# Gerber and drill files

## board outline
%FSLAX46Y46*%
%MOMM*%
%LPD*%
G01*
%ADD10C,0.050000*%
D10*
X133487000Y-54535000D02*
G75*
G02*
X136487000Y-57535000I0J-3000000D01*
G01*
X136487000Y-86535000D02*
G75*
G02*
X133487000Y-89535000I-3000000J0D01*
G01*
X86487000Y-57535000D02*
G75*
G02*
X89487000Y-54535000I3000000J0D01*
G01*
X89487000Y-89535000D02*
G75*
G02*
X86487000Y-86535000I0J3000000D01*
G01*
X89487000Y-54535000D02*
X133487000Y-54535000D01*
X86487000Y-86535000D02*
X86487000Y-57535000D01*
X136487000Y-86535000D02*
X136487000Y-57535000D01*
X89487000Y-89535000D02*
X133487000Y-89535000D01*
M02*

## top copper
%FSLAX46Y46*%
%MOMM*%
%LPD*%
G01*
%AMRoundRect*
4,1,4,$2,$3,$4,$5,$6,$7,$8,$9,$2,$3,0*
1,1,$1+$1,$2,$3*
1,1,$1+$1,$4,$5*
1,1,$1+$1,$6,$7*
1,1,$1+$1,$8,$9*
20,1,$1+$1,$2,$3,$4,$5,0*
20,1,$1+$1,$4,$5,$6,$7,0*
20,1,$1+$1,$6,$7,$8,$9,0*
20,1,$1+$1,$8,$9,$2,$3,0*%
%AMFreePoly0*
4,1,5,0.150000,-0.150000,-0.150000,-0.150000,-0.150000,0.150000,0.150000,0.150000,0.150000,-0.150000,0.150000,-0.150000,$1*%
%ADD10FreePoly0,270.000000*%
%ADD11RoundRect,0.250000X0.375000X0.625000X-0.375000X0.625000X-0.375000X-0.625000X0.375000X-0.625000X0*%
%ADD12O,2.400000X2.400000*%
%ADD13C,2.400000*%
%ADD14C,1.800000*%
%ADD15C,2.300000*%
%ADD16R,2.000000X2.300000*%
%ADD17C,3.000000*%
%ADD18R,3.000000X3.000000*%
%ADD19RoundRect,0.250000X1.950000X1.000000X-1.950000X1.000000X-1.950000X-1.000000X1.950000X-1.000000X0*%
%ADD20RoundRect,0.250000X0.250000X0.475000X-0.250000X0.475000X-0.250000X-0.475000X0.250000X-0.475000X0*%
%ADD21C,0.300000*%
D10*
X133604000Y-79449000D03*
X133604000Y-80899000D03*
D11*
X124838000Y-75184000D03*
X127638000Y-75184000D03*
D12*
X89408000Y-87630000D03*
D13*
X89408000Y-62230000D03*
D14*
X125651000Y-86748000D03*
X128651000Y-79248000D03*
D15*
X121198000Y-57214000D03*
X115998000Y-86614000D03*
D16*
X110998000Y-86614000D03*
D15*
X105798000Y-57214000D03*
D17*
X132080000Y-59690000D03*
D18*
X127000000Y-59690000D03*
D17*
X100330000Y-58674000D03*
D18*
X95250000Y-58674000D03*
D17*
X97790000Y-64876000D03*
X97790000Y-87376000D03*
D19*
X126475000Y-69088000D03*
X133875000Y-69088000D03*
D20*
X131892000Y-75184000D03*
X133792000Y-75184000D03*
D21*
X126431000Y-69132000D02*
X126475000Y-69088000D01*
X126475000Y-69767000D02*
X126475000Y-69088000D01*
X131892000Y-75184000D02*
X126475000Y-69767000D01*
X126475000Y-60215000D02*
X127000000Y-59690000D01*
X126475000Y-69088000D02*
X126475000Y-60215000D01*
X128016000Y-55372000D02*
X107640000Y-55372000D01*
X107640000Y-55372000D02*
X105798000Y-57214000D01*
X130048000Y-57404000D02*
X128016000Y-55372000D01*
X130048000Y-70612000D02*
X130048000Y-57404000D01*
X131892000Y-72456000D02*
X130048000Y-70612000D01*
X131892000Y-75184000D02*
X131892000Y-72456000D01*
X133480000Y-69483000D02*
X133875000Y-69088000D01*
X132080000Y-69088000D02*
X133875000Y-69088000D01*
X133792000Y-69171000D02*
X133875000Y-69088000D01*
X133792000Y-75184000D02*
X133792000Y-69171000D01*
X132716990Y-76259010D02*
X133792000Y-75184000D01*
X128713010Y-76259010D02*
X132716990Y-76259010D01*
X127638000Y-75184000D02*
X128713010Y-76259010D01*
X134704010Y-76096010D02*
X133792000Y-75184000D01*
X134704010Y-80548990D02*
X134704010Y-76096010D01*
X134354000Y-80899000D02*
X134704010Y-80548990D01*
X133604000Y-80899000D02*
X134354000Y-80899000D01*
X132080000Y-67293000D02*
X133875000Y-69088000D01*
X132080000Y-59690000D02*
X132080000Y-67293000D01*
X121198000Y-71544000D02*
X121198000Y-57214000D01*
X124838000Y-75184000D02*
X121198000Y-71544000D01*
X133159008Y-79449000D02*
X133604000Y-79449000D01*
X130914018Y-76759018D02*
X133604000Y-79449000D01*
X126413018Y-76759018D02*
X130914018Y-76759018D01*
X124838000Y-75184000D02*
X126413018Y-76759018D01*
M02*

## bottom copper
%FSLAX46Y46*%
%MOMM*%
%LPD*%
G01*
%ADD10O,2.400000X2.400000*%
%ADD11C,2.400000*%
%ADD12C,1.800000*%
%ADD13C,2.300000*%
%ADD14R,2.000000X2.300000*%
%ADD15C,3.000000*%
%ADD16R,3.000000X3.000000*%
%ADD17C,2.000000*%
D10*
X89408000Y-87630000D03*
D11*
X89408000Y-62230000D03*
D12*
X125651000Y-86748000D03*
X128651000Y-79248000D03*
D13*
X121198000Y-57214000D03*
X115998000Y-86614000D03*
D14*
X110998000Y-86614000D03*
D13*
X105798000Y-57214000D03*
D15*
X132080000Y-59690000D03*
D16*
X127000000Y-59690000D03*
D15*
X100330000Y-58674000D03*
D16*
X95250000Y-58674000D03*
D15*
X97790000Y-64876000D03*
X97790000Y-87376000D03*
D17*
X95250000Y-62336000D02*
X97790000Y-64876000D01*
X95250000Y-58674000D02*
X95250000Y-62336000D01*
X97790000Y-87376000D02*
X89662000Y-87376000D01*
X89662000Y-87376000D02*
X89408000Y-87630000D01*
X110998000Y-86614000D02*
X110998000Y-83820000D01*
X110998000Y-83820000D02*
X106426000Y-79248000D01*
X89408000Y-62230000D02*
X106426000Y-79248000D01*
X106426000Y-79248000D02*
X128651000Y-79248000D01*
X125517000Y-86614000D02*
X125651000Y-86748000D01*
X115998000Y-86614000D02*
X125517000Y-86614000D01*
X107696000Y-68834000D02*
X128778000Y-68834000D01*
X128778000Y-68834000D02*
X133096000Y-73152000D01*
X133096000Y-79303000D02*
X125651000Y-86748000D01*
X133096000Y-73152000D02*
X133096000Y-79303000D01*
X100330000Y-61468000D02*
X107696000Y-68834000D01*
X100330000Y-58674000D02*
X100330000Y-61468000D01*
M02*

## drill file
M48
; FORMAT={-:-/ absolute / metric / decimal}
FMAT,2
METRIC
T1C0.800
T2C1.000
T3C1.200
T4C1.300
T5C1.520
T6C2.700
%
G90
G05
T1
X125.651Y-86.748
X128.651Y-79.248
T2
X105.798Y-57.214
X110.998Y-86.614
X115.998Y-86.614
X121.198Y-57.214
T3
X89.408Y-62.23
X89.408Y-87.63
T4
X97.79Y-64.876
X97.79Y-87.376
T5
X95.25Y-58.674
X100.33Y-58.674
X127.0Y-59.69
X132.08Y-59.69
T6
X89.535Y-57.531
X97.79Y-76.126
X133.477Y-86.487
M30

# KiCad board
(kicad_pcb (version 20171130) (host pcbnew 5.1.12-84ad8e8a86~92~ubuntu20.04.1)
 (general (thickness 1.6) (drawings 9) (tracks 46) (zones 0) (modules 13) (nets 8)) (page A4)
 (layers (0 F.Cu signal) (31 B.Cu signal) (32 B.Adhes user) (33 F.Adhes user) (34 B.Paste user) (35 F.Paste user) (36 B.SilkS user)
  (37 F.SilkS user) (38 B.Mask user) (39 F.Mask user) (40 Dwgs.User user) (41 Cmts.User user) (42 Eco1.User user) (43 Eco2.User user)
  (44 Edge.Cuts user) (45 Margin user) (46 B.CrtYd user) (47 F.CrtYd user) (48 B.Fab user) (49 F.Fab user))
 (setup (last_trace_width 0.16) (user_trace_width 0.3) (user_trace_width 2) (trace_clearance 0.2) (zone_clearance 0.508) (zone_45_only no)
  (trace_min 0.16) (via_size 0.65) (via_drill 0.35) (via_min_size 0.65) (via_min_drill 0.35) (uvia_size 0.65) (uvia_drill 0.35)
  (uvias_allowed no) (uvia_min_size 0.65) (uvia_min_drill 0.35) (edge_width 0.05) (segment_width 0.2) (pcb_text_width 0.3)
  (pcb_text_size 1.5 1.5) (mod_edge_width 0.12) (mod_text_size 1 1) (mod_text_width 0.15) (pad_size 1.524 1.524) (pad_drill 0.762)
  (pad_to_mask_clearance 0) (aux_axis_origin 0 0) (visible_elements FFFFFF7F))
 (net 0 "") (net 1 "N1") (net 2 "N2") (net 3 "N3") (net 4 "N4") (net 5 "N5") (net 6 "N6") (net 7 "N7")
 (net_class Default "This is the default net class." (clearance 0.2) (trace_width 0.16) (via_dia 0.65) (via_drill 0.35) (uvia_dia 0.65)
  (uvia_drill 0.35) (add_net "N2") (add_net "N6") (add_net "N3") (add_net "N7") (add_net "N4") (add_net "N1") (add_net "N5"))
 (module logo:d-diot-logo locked (layer B.Cu) (at 112.522 69.596 180)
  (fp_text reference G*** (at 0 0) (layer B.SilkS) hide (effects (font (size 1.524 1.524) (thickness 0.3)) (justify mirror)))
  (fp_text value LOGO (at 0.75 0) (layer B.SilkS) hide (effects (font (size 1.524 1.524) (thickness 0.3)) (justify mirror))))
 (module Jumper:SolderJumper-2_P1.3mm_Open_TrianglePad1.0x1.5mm (layer F.Cu) (at 133.604 80.174 270)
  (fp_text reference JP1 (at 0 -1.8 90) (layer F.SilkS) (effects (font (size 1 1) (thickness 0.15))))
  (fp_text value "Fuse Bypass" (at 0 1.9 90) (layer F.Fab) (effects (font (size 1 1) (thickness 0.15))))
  (pad 1 smd custom (at -0.725 0 270) (size 0.3 0.3) (layers F.Cu F.Mask) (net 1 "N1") (zone_connect 2)
   (options (clearance outline) (anchor rect)) (primitives))
  (pad 2 smd custom (at 0.725 0 270) (size 0.3 0.3) (layers F.Cu F.Mask) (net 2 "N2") (zone_connect 2)
   (options (clearance outline) (anchor rect)) (primitives)))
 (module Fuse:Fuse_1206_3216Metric (layer F.Cu) (at 126.238 75.184 180)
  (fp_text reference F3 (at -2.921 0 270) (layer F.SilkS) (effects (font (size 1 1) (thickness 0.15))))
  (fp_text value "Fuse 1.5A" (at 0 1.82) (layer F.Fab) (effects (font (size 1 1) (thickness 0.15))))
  (pad 2 smd roundrect (at 1.4 0 180) (size 1.25 1.75) (layers F.Cu F.Paste F.Mask) (roundrect_rratio 0.2) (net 1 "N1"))
  (pad 1 smd roundrect (at -1.4 0 180) (size 1.25 1.75) (layers F.Cu F.Paste F.Mask) (roundrect_rratio 0.2) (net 2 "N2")))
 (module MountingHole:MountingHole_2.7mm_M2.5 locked (layer F.Cu) (at 133.477 86.487 90)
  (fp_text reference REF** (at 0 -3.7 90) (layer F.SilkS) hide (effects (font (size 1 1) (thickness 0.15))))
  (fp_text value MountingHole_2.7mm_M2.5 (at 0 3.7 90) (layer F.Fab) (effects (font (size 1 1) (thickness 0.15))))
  (pad 1 np_thru_hole circle (at 0 0 90) (size 2.7 2.7) (drill 2.7) (layers *.Cu *.Mask)))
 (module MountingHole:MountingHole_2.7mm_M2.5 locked (layer F.Cu) (at 89.535 57.531 90)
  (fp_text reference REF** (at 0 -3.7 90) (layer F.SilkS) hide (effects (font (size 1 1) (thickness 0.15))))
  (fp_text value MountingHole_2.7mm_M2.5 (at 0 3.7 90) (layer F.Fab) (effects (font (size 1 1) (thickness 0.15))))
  (pad 1 np_thru_hole circle (at 0 0 90) (size 2.7 2.7) (drill 2.7) (layers *.Cu *.Mask)))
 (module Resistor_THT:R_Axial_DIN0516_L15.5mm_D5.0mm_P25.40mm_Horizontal (layer F.Cu) (at 89.408 62.23 270)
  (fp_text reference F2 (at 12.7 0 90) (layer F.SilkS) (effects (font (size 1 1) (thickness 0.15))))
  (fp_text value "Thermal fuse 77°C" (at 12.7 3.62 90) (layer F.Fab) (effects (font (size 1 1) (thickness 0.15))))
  (pad 2 thru_hole oval (at 25.4 0 270) (size 2.4 2.4) (drill 1.2) (layers *.Cu *.Mask) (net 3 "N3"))
  (pad 1 thru_hole circle (at 0 0 270) (size 2.4 2.4) (drill 1.2) (layers *.Cu *.Mask) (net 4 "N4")))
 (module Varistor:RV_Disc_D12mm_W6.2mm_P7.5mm (layer F.Cu) (at 128.651 79.248 270)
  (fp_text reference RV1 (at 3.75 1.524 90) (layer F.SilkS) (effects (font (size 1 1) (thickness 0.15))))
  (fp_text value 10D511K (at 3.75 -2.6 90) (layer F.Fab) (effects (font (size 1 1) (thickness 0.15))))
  (pad 2 thru_hole circle (at 7.5 3 270) (size 1.8 1.8) (drill 0.8) (layers *.Cu *.Mask) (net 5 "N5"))
  (pad 1 thru_hole circle (at 0 0 270) (size 1.8 1.8) (drill 0.8) (layers *.Cu *.Mask) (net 4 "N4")))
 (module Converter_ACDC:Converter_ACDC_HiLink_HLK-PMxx (layer F.Cu) (at 110.998 86.614 90)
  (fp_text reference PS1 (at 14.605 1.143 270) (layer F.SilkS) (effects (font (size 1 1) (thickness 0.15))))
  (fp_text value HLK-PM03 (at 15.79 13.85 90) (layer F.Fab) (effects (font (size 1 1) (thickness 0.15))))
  (pad 4 thru_hole circle (at 29.4 10.2 90) (size 2.3 2.3) (drill 1) (layers *.Cu *.Mask) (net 1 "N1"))
  (pad 2 thru_hole circle (at 0 5 90) (size 2.3 2.3) (drill 1) (layers *.Cu *.Mask) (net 5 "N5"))
  (pad 1 thru_hole rect (at 0 0 90) (size 2.3 2) (drill 1) (layers *.Cu *.Mask) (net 4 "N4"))
  (pad 3 thru_hole circle (at 29.4 -5.2 90) (size 2.3 2.3) (drill 1) (layers *.Cu *.Mask) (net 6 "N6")))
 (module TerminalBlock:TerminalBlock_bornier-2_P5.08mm (layer F.Cu) (at 127 59.69)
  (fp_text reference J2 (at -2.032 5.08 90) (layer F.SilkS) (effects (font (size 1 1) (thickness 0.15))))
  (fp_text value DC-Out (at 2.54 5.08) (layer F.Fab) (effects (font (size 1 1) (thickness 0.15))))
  (pad 2 thru_hole circle (at 5.08 0) (size 3 3) (drill 1.52) (layers *.Cu *.Mask) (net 2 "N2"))
  (pad 1 thru_hole rect (at 0 0) (size 3 3) (drill 1.52) (layers *.Cu *.Mask) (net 6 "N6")))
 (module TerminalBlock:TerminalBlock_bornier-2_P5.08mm (layer F.Cu) (at 95.25 58.674)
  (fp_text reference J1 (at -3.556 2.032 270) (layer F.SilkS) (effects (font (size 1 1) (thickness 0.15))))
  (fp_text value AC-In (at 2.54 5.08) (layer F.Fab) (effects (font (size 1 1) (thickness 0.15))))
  (pad 2 thru_hole circle (at 5.08 0) (size 3 3) (drill 1.52) (layers *.Cu *.Mask) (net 5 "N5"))
  (pad 1 thru_hole rect (at 0 0) (size 3 3) (drill 1.52) (layers *.Cu *.Mask) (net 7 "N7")))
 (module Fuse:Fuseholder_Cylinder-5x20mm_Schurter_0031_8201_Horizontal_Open (layer F.Cu) (at 97.79 87.376 90)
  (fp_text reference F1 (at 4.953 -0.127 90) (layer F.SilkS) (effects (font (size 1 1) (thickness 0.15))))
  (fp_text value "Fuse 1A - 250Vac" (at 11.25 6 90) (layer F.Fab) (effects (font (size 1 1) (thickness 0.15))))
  (pad "" np_thru_hole circle (at 11.25 0 90) (size 2.7 2.7) (drill 2.7) (layers *.Cu *.Mask))
  (pad 2 thru_hole circle (at 22.5 0 90) (size 3 3) (drill 1.3) (layers *.Cu *.Mask) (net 7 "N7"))
  (pad 1 thru_hole circle (at 0 0 90) (size 3 3) (drill 1.3) (layers *.Cu *.Mask) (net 3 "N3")))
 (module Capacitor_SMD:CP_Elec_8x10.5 (layer F.Cu) (at 130.175 69.088 180)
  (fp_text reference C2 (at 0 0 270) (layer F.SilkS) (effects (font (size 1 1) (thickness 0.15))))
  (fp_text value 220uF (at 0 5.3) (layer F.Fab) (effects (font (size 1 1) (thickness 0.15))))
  (pad 2 smd roundrect (at 3.7 0 180) (size 4.4 2.5) (layers F.Cu F.Paste F.Mask) (roundrect_rratio 0.1) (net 6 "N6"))
  (pad 1 smd roundrect (at -3.7 0 180) (size 4.4 2.5) (layers F.Cu F.Paste F.Mask) (roundrect_rratio 0.1) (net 2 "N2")))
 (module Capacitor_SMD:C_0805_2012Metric (layer F.Cu) (at 132.842 75.184 180)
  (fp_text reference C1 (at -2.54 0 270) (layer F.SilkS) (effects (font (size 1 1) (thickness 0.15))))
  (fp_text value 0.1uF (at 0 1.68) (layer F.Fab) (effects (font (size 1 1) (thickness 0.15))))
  (pad 2 smd roundrect (at 0.95 0 180) (size 1 1.45) (layers F.Cu F.Paste F.Mask) (roundrect_rratio 0.25) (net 6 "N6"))
  (pad 1 smd roundrect (at -0.95 0 180) (size 1 1.45) (layers F.Cu F.Paste F.Mask) (roundrect_rratio 0.25) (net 2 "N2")))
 (gr_arc (start 133.487 57.535) (end 136.487 57.535) (angle -90) (layer Edge.Cuts) (width 0.05))
 (gr_arc (start 133.487 86.535) (end 133.487 89.535) (angle -90) (layer Edge.Cuts) (width 0.05))
 (gr_arc (start 89.487 57.535) (end 89.487 54.535) (angle -90) (layer Edge.Cuts) (width 0.05))
 (gr_arc (start 89.487 86.535) (end 86.487 86.535) (angle -90) (layer Edge.Cuts) (width 0.05))
 (gr_line (start 89.487 54.535) (end 133.487 54.535) (layer Edge.Cuts) (width 0.05))
 (gr_line (start 86.487 86.535) (end 86.487 57.535) (layer Edge.Cuts) (width 0.05))
 (gr_line (start 136.487 86.535) (end 136.487 57.535) (layer Edge.Cuts) (width 0.05))
 (gr_line (start 89.487 89.535) (end 133.487 89.535) (layer Edge.Cuts) (width 0.05))
 (segment (start 126.431 69.132) (end 126.475 69.088) (width 0.3) (layer F.Cu) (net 6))
 (segment (start 126.475 69.767) (end 126.475 69.088) (width 0.3) (layer F.Cu) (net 6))
 (segment (start 131.892 75.184) (end 126.475 69.767) (width 0.3) (layer F.Cu) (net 6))
 (segment (start 126.475 60.215) (end 127 59.69) (width 0.3) (layer F.Cu) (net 6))
 (segment (start 126.475 69.088) (end 126.475 60.215) (width 0.3) (layer F.Cu) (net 6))
 (segment (start 128.016 55.372) (end 107.64 55.372) (width 0.3) (layer F.Cu) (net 6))
 (segment (start 107.64 55.372) (end 105.798 57.214) (width 0.3) (layer F.Cu) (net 6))
 (segment (start 130.048 57.404) (end 128.016 55.372) (width 0.3) (layer F.Cu) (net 6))
 (segment (start 130.048 70.612) (end 130.048 57.404) (width 0.3) (layer F.Cu) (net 6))
 (segment (start 131.892 72.456) (end 130.048 70.612) (width 0.3) (layer F.Cu) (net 6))
 (segment (start 131.892 75.184) (end 131.892 72.456) (width 0.3) (layer F.Cu) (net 6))
 (segment (start 133.48 69.483) (end 133.875 69.088) (width 0.3) (layer F.Cu) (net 2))
 (segment (start 132.08 69.088) (end 133.875 69.088) (width 0.3) (layer F.Cu) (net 2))
 (segment (start 133.792 69.171) (end 133.875 69.088) (width 0.3) (layer F.Cu) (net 2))
 (segment (start 133.792 75.184) (end 133.792 69.171) (width 0.3) (layer F.Cu) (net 2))
 (segment (start 132.71699 76.25901) (end 133.792 75.184) (width 0.3) (layer F.Cu) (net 2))
 (segment (start 128.71301 76.25901) (end 132.71699 76.25901) (width 0.3) (layer F.Cu) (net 2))
 (segment (start 127.638 75.184) (end 128.71301 76.25901) (width 0.3) (layer F.Cu) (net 2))
 (segment (start 134.70401 76.09601) (end 133.792 75.184) (width 0.3) (layer F.Cu) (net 2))
 (segment (start 134.70401 80.54899) (end 134.70401 76.09601) (width 0.3) (layer F.Cu) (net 2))
 (segment (start 134.354 80.899) (end 134.70401 80.54899) (width 0.3) (layer F.Cu) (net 2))
 (segment (start 133.604 80.899) (end 134.354 80.899) (width 0.3) (layer F.Cu) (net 2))
 (segment (start 132.08 67.293) (end 133.875 69.088) (width 0.3) (layer F.Cu) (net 2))
 (segment (start 132.08 59.69) (end 132.08 67.293) (width 0.3) (layer F.Cu) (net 2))
 (segment (start 95.25 62.336) (end 97.79 64.876) (width 2) (layer B.Cu) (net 7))
 (segment (start 95.25 58.674) (end 95.25 62.336) (width 2) (layer B.Cu) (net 7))
 (segment (start 97.79 87.376) (end 89.662 87.376) (width 2) (layer B.Cu) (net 3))
 (segment (start 89.662 87.376) (end 89.408 87.63) (width 2) (layer B.Cu) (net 3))
 (segment (start 110.998 86.614) (end 110.998 83.82) (width 2) (layer B.Cu) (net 4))
 (segment (start 110.998 83.82) (end 106.426 79.248) (width 2) (layer B.Cu) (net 4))
 (segment (start 89.408 62.23) (end 106.426 79.248) (width 2) (layer B.Cu) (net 4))
 (segment (start 106.426 79.248) (end 128.651 79.248) (width 2) (layer B.Cu) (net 4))
 (segment (start 121.198 71.544) (end 121.198 57.214) (width 0.3) (layer F.Cu) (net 1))
 (segment (start 124.838 75.184) (end 121.198 71.544) (width 0.3) (layer F.Cu) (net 1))
 (segment (start 133.159008 79.449) (end 133.604 79.449) (width 0.3) (layer F.Cu) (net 1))
 (segment (start 130.914018 76.759018) (end 133.604 79.449) (width 0.3) (layer F.Cu) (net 1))
 (segment (start 126.413018 76.759018) (end 130.914018 76.759018) (width 0.3) (layer F.Cu) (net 1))
 (segment (start 124.838 75.184) (end 126.413018 76.759018) (width 0.3) (layer F.Cu) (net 1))
 (segment (start 125.517 86.614) (end 125.651 86.748) (width 2) (layer B.Cu) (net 5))
 (segment (start 115.998 86.614) (end 125.517 86.614) (width 2) (layer B.Cu) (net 5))
 (segment (start 107.696 68.834) (end 128.778 68.834) (width 2) (layer B.Cu) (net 5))
 (segment (start 128.778 68.834) (end 133.096 73.152) (width 2) (layer B.Cu) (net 5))
 (segment (start 133.096 79.303) (end 125.651 86.748) (width 2) (layer B.Cu) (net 5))
 (segment (start 133.096 73.152) (end 133.096 79.303) (width 2) (layer B.Cu) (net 5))
 (segment (start 100.33 61.468) (end 107.696 68.834) (width 2) (layer B.Cu) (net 5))
 (segment (start 100.33 58.674) (end 100.33 61.468) (width 2) (layer B.Cu) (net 5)))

